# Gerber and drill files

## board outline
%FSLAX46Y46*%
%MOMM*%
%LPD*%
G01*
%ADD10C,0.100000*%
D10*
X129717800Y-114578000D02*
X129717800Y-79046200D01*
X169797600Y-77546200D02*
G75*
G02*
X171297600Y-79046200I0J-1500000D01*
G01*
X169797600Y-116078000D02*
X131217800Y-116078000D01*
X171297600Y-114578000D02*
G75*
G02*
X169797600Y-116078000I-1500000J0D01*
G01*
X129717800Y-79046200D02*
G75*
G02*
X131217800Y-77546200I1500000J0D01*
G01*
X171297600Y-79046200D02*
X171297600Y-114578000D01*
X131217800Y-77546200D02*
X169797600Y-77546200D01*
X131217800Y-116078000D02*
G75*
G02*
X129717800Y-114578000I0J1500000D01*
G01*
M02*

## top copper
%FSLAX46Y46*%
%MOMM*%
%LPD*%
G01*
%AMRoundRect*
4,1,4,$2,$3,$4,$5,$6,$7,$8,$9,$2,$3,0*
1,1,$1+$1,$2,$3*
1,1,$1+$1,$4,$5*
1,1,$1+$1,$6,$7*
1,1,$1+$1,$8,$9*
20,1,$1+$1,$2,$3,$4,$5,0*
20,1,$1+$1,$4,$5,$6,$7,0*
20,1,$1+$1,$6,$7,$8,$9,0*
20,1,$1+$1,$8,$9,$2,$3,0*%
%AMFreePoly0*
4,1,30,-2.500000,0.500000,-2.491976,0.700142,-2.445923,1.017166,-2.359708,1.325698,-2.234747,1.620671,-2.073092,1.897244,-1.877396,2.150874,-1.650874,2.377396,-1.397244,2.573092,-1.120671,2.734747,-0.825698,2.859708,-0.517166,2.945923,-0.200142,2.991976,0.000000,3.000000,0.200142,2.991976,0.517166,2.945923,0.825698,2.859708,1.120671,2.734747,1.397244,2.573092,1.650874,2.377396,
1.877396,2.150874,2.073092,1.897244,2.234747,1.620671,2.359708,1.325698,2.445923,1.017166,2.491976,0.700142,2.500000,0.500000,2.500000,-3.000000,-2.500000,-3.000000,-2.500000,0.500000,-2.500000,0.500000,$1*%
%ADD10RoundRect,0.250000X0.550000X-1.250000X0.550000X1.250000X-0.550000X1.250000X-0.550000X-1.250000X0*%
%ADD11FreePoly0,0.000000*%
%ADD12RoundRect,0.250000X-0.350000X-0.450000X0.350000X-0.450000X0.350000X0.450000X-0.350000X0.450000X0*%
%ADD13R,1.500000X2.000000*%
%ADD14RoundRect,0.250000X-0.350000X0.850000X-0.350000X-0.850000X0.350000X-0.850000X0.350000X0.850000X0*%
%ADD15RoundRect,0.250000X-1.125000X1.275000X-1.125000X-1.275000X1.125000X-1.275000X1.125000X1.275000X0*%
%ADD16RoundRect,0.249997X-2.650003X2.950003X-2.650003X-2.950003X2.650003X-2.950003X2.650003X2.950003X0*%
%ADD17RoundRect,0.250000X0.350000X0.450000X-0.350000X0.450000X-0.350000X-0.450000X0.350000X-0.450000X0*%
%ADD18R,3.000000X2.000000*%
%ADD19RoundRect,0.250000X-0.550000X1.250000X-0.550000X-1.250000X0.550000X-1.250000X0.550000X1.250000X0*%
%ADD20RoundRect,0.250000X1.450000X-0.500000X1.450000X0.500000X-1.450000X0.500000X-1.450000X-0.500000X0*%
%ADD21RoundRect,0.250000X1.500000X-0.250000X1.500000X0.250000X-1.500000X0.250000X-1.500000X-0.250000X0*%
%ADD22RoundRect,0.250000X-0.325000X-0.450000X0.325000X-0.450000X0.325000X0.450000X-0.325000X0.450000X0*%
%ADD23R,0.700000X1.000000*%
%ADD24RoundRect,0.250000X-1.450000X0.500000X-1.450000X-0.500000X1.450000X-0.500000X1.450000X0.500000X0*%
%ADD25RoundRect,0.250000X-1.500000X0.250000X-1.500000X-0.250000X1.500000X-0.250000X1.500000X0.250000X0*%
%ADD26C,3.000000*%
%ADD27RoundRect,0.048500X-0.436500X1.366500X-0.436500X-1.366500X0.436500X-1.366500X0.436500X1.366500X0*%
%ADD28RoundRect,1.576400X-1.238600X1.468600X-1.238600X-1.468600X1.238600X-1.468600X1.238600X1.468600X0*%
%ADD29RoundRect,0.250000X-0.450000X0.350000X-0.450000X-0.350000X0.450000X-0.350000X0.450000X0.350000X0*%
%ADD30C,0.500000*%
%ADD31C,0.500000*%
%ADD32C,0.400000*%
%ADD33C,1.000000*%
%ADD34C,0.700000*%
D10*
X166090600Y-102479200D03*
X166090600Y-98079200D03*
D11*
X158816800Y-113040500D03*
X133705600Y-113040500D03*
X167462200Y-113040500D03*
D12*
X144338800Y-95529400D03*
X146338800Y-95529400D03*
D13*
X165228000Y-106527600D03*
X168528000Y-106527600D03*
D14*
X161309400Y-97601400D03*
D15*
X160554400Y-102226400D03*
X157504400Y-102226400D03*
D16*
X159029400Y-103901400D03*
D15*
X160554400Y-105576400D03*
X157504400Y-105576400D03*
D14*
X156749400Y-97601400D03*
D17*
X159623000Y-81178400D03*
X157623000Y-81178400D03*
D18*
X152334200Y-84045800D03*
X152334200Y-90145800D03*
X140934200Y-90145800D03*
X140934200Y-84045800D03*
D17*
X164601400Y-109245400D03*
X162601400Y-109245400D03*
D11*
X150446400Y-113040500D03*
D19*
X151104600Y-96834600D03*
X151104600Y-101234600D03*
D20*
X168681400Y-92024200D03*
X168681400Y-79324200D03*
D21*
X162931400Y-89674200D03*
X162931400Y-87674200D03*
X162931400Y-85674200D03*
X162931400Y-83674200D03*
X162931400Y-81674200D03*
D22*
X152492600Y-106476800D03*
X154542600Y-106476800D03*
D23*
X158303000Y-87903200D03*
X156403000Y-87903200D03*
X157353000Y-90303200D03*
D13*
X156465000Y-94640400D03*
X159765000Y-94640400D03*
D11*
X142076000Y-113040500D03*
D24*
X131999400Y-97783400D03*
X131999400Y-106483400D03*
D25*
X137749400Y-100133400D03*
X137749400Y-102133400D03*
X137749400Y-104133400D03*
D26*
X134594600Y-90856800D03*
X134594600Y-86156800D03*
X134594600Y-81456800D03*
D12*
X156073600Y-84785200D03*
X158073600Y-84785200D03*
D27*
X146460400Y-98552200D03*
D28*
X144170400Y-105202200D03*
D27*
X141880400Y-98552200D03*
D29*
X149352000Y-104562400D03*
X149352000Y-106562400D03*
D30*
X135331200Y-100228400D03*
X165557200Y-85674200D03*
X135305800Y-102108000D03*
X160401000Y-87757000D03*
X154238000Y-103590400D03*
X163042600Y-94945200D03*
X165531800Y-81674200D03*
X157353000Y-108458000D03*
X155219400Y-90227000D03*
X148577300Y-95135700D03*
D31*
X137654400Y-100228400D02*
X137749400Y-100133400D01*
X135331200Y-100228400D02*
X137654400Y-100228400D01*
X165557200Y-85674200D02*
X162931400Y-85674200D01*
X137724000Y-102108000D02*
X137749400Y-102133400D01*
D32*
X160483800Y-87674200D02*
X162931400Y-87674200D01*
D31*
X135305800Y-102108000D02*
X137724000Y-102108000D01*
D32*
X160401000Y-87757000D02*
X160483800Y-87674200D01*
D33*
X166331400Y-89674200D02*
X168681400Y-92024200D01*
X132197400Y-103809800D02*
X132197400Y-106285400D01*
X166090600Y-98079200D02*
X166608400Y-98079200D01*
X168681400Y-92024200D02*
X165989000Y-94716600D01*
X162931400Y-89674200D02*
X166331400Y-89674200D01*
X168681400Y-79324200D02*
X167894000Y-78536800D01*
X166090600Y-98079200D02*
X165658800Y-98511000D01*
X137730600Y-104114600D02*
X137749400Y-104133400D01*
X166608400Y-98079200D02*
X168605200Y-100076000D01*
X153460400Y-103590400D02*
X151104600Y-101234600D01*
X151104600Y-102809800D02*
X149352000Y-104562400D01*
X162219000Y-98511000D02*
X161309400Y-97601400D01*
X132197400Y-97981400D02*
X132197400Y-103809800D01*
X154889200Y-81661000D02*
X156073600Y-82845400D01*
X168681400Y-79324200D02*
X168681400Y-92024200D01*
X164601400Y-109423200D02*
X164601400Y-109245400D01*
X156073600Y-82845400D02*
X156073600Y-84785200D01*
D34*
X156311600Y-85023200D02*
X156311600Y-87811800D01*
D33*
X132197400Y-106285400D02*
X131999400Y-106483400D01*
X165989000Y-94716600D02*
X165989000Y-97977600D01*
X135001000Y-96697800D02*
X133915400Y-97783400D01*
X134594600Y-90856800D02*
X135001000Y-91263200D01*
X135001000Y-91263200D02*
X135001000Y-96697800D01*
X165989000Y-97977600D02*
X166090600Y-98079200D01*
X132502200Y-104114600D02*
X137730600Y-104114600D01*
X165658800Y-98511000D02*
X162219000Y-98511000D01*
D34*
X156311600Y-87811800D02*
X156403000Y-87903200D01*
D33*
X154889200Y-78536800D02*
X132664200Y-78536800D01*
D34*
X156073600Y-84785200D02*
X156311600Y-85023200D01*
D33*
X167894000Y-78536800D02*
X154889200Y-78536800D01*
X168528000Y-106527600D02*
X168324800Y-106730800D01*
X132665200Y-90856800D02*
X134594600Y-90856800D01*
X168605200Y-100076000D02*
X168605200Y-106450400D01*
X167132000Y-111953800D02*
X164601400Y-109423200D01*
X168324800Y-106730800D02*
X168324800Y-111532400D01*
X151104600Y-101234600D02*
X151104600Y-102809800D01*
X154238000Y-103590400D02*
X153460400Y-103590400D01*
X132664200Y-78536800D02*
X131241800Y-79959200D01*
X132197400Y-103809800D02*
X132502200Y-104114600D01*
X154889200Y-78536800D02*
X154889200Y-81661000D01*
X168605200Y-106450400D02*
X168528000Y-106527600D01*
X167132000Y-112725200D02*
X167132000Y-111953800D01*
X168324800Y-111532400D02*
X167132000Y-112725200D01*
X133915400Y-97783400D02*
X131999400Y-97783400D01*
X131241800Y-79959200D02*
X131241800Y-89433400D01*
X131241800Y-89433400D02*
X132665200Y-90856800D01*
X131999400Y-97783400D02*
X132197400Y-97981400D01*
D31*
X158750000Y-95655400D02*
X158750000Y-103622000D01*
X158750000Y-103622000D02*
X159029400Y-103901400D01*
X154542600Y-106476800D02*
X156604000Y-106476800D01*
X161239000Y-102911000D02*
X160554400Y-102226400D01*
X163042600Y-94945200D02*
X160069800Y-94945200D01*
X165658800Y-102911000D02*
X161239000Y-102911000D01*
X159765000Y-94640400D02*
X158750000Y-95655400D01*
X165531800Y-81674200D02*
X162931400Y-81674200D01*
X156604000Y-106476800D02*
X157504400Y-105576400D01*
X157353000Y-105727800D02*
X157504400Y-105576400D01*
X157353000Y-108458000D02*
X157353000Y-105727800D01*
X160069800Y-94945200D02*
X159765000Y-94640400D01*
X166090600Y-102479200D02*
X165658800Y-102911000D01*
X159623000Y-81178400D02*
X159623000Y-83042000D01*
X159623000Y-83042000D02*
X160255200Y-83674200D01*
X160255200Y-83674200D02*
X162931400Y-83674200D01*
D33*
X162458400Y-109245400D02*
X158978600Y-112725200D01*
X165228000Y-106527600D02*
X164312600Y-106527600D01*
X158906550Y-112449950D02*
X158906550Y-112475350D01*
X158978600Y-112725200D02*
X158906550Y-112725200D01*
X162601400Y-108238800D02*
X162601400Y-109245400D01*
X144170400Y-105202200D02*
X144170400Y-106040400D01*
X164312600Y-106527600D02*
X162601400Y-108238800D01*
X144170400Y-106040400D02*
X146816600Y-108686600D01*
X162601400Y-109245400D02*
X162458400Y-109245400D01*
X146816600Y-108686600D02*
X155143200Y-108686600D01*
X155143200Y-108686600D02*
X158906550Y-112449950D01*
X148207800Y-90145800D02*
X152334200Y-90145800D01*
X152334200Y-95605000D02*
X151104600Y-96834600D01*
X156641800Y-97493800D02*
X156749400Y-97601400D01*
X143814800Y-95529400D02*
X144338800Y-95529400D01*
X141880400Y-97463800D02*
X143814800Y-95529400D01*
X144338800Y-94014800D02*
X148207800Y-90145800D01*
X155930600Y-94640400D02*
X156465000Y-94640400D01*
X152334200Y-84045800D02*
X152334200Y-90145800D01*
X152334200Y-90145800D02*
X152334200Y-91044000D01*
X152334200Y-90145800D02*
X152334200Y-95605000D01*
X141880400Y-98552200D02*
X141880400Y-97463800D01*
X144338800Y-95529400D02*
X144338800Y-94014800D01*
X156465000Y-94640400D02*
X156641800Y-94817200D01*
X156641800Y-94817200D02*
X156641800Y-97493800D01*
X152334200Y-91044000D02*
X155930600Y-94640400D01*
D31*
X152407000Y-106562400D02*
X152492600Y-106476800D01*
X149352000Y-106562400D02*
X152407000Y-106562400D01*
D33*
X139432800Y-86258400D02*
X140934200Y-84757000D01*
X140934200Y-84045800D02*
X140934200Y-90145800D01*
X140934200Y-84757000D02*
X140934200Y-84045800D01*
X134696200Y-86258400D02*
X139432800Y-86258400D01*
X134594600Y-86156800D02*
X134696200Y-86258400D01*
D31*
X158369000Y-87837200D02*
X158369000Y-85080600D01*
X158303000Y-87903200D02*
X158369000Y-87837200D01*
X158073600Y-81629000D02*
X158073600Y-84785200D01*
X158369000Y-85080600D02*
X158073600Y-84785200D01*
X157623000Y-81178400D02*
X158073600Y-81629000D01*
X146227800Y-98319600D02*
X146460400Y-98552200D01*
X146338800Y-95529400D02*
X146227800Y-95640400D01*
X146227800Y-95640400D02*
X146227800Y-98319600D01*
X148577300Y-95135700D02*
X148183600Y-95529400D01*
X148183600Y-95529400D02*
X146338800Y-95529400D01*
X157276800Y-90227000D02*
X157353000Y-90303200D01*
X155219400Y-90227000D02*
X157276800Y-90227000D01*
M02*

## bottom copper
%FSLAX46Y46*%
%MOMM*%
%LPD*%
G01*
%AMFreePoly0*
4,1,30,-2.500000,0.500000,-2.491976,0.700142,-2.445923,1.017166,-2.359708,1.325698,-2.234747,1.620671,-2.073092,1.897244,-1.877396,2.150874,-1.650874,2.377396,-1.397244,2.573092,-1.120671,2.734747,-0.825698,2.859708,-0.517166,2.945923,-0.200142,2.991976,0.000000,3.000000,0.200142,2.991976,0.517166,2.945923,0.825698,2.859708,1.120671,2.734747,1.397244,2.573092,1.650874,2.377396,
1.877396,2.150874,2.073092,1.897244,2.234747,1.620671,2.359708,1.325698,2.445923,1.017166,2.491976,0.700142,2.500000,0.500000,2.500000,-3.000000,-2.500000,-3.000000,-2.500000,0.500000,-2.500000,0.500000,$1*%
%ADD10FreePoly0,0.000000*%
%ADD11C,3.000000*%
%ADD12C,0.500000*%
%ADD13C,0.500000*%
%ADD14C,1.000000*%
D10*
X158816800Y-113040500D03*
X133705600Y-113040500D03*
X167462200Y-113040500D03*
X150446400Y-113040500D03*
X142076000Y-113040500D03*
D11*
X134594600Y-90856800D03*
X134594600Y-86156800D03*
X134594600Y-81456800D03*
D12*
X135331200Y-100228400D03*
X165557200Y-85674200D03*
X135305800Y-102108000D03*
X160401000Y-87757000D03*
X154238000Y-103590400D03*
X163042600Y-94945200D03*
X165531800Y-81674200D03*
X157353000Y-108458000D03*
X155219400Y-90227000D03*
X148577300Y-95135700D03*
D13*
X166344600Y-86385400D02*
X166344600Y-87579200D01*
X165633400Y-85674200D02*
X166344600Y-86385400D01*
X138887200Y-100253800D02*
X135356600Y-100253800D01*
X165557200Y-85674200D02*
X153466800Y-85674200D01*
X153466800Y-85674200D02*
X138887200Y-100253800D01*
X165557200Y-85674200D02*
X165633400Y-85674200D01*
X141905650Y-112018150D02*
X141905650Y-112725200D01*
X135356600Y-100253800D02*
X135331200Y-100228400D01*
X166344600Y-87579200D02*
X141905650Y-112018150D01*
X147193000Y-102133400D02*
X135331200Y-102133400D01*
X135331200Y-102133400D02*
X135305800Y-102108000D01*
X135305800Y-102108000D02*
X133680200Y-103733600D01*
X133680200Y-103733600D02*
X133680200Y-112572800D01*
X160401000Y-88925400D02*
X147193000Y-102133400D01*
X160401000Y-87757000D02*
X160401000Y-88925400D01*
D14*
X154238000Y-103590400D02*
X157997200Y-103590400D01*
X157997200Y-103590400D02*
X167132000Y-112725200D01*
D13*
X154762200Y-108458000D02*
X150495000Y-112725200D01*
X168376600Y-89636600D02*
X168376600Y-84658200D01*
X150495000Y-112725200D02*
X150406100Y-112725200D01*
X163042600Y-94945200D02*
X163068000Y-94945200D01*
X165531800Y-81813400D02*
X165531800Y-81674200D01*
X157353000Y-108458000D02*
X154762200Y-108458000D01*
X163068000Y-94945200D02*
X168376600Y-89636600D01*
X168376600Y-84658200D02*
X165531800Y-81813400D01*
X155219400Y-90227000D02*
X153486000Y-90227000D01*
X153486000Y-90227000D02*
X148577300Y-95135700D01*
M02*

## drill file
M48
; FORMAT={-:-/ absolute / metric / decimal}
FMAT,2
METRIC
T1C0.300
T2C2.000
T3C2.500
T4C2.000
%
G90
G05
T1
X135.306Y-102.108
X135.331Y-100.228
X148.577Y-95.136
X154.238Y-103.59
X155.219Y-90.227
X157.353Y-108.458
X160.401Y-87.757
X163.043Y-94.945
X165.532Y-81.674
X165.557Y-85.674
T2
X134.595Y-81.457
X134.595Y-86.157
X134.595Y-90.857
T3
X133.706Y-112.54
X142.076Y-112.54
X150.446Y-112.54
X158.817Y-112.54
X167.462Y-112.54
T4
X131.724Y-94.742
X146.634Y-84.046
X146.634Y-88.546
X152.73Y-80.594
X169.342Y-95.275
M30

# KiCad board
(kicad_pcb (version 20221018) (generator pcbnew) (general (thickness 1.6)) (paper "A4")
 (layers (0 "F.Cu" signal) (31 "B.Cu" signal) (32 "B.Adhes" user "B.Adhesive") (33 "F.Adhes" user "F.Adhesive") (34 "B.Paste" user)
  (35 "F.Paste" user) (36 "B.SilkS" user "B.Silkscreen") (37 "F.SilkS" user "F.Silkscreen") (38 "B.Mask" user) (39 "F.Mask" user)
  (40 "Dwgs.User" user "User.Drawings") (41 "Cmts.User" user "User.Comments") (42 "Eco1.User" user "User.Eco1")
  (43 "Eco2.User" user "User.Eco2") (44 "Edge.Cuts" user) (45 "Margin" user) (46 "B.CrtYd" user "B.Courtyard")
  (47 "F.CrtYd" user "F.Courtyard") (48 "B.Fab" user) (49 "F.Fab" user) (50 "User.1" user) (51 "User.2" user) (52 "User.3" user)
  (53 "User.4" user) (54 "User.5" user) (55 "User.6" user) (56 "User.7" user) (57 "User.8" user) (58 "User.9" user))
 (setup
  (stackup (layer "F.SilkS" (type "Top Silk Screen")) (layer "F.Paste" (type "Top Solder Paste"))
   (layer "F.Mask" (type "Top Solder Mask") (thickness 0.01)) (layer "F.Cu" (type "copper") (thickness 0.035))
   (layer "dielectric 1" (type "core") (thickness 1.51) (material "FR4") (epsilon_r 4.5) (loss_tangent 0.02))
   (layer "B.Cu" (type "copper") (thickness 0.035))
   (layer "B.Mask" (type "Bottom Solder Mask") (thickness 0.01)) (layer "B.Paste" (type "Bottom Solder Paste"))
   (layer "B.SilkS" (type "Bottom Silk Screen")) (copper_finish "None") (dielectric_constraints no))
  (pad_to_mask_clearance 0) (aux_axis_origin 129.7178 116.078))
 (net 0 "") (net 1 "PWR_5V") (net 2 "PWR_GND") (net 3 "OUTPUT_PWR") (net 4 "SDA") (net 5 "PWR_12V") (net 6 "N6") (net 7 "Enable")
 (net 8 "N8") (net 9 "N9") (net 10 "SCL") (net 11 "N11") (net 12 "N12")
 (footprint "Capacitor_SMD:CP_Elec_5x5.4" (layer "F.Cu") (at 166.0906 100.2792 90)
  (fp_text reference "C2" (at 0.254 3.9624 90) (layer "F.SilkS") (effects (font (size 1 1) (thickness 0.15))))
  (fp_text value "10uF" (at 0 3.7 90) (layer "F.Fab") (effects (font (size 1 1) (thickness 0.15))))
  (pad "1" smd roundrect (at -2.2 0 90) (size 3 1.6) (layers "F.Cu" "F.Paste" "F.Mask") (roundrect_rratio 0.15625) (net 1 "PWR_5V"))
  (pad "2" smd roundrect (at 2.2 0 90) (size 3 1.6) (layers "F.Cu" "F.Paste" "F.Mask") (roundrect_rratio 0.15625) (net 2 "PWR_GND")))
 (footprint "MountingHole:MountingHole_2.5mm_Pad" (layer "F.Cu") (at 158.8168 112.5405)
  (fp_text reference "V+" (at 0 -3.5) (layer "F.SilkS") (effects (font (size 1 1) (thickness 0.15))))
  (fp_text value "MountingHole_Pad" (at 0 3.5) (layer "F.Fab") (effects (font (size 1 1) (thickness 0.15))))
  (pad "1" thru_hole roundrect (at 0 0) (size 5 6) (drill 2.5 (offset 0 0.5)) (layers "*.Cu" "*.Mask") (roundrect_rratio 0.5)
   (chamfer_ratio 0) (chamfer bottom_left bottom_right) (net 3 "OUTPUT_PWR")))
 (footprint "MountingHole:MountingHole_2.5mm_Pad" (layer "F.Cu") (at 133.7056 112.5405)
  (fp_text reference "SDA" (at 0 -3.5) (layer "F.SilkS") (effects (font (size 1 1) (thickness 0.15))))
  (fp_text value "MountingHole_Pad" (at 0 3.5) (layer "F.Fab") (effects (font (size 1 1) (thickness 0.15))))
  (pad "1" thru_hole roundrect (at 0 0) (size 5 6) (drill 2.5 (offset 0 0.5)) (layers "*.Cu" "*.Mask") (roundrect_rratio 0.5)
   (chamfer_ratio 0) (chamfer bottom_left bottom_right) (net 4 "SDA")))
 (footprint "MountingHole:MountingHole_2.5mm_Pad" (layer "F.Cu") (at 167.4622 112.5405)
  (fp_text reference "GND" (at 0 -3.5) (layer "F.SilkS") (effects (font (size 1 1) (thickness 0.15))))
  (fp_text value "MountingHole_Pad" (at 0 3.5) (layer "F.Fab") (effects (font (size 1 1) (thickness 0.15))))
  (pad "1" thru_hole roundrect (at 0 0) (size 5 6) (drill 2.5 (offset 0 0.5)) (layers "*.Cu" "*.Mask") (roundrect_rratio 0.5)
   (chamfer_ratio 0) (chamfer bottom_left bottom_right) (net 2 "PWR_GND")))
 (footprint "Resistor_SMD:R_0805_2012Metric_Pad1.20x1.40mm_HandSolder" (layer "F.Cu") (at 145.3388 95.5294)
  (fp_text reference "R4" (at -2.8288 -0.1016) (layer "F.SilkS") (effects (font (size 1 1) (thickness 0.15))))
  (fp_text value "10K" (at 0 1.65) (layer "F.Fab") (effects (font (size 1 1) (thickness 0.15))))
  (pad "1" smd roundrect (at -1 0) (size 1.2 1.4) (layers "F.Cu" "F.Paste" "F.Mask") (roundrect_rratio 0.2083333333) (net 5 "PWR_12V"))
  (pad "2" smd roundrect (at 1 0) (size 1.2 1.4) (layers "F.Cu" "F.Paste" "F.Mask") (roundrect_rratio 0.2083333333) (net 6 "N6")))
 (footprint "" (layer "F.Cu") (at 131.7244 94.742)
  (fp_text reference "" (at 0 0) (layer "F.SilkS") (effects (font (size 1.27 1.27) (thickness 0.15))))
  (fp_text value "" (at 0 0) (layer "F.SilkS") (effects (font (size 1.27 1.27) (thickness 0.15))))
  (pad "" np_thru_hole circle (at 0 0) (size 2 2) (drill 2) (layers "F&B.Cu" "*.Mask")))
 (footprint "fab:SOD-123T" (layer "F.Cu") (at 166.878 106.5276)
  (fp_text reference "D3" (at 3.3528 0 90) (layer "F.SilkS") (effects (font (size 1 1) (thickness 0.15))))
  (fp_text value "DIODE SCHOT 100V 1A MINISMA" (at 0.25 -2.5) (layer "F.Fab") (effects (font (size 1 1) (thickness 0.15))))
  (pad "1" smd rect (at -1.65 0) (size 1.5 2) (layers "F.Cu" "F.Paste" "F.Mask") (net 3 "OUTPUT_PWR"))
  (pad "2" smd rect (at 1.65 0) (size 1.5 2) (layers "F.Cu" "F.Paste" "F.Mask") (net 2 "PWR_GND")))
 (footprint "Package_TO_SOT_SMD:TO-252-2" (layer "F.Cu") (at 159.0294 102.6414 -90)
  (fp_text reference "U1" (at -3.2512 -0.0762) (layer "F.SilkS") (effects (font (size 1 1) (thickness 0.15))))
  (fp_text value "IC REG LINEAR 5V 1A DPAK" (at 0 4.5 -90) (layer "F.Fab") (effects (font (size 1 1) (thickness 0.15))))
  (pad "1" smd roundrect (at -5.04 -2.28 270) (size 2.2 1.2) (layers "F.Cu" "F.Paste" "F.Mask") (roundrect_rratio 0.2083333333)
   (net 2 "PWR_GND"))
  (pad "2" smd roundrect (at -0.415 -1.525 270) (size 3.05 2.75) (layers "F.Cu" "F.Paste") (roundrect_rratio 0.09090909091) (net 1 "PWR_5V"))
  (pad "2" smd roundrect (at -0.415 1.525 270) (size 3.05 2.75) (layers "F.Cu" "F.Paste") (roundrect_rratio 0.09090909091) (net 1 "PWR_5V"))
  (pad "2" smd roundrect (at 1.26 0 270) (size 6.4 5.8) (layers "F.Cu" "F.Mask") (roundrect_rratio 0.04310293103) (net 1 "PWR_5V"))
  (pad "2" smd roundrect (at 2.935 -1.525 270) (size 3.05 2.75) (layers "F.Cu" "F.Paste") (roundrect_rratio 0.09090909091) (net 1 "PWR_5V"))
  (pad "2" smd roundrect (at 2.935 1.525 270) (size 3.05 2.75) (layers "F.Cu" "F.Paste") (roundrect_rratio 0.09090909091) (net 1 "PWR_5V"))
  (pad "3" smd roundrect (at -5.04 2.28 270) (size 2.2 1.2) (layers "F.Cu" "F.Paste" "F.Mask") (roundrect_rratio 0.2083333333)
   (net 5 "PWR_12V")))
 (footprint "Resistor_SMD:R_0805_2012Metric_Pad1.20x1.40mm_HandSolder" (layer "F.Cu") (at 158.623 81.1784 180)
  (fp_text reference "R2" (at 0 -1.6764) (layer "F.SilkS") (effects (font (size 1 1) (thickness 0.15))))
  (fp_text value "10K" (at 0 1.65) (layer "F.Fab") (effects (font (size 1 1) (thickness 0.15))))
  (pad "1" smd roundrect (at -1 0 180) (size 1.2 1.4) (layers "F.Cu" "F.Paste" "F.Mask") (roundrect_rratio 0.2083333333) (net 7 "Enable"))
  (pad "2" smd roundrect (at 1 0 180) (size 1.2 1.4) (layers "F.Cu" "F.Paste" "F.Mask") (roundrect_rratio 0.2083333333) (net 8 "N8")))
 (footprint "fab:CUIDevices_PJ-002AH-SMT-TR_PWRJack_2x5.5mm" (layer "F.Cu") (at 146.6342 87.0458 -90)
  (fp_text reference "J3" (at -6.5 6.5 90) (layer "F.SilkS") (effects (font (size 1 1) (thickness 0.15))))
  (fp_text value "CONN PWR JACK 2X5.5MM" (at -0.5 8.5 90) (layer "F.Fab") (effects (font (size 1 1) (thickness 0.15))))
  (pad "" np_thru_hole circle (at -3 0) (size 2 2) (drill 2) (layers "F&B.Cu" "*.Mask"))
  (pad "" np_thru_hole circle (at 1.5 0) (size 2 2) (drill 2) (layers "F&B.Cu" "*.Mask"))
  (pad "1" smd rect (at -3 -5.7) (size 3 2) (layers "F.Cu" "F.Paste" "F.Mask") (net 5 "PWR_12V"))
  (pad "1" smd rect (at 3.1 -5.7) (size 3 2) (layers "F.Cu" "F.Paste" "F.Mask") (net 5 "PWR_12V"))
  (pad "2" smd rect (at 3.1 5.7) (size 3 2) (layers "F.Cu" "F.Paste" "F.Mask") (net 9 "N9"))
  (pad "3" smd rect (at -3 5.7) (size 3 2) (layers "F.Cu" "F.Paste" "F.Mask") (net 9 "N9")))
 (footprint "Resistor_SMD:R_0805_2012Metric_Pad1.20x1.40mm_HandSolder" (layer "F.Cu") (at 163.6014 109.2454 180)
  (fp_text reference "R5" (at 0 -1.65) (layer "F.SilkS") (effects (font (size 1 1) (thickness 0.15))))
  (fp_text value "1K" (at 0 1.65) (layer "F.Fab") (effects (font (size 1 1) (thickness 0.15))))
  (pad "1" smd roundrect (at -1 0 180) (size 1.2 1.4) (layers "F.Cu" "F.Paste" "F.Mask") (roundrect_rratio 0.2083333333) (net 2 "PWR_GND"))
  (pad "2" smd roundrect (at 1 0 180) (size 1.2 1.4) (layers "F.Cu" "F.Paste" "F.Mask") (roundrect_rratio 0.2083333333) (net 3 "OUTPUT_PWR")))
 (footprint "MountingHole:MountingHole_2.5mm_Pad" (layer "F.Cu") (at 150.4464 112.5405)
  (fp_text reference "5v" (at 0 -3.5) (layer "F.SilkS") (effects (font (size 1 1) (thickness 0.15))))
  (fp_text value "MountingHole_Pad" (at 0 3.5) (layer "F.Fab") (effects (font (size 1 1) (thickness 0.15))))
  (pad "1" thru_hole roundrect (at 0 0) (size 5 6) (drill 2.5 (offset 0 0.5)) (layers "*.Cu" "*.Mask") (roundrect_rratio 0.5)
   (chamfer_ratio 0) (chamfer bottom_left bottom_right) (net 1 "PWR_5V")))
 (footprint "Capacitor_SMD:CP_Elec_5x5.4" (layer "F.Cu") (at 151.1046 99.0346 -90)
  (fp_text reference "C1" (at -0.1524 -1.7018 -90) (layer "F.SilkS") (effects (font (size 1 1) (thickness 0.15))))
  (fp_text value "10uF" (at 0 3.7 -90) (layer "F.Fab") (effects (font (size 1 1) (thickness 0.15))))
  (pad "1" smd roundrect (at -2.2 0 270) (size 3 1.6) (layers "F.Cu" "F.Paste" "F.Mask") (roundrect_rratio 0.15625) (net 5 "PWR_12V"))
  (pad "2" smd roundrect (at 2.2 0 270) (size 3 1.6) (layers "F.Cu" "F.Paste" "F.Mask") (roundrect_rratio 0.15625) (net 2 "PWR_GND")))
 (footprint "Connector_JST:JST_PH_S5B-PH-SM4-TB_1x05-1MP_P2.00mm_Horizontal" (layer "F.Cu") (at 165.7814 85.6742 90)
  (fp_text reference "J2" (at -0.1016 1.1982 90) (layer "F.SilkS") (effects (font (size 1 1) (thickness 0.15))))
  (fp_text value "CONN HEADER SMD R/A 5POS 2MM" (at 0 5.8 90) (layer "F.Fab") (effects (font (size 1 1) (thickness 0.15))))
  (pad "" smd roundrect (at -6.35 2.9 90) (size 1.5 3.4) (layers "F.Cu" "F.Paste" "F.Mask") (roundrect_rratio 0.1666666667)
   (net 2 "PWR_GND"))
  (pad "" smd roundrect (at 6.35 2.9 90) (size 1.5 3.4) (layers "F.Cu" "F.Paste" "F.Mask") (roundrect_rratio 0.1666666667) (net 2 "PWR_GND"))
  (pad "1" smd roundrect (at -4 -2.85 90) (size 1 3.5) (layers "F.Cu" "F.Paste" "F.Mask") (roundrect_rratio 0.25) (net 2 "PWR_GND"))
  (pad "2" smd roundrect (at -2 -2.85 90) (size 1 3.5) (layers "F.Cu" "F.Paste" "F.Mask") (roundrect_rratio 0.25) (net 4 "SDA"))
  (pad "3" smd roundrect (at 0 -2.85 90) (size 1 3.5) (layers "F.Cu" "F.Paste" "F.Mask") (roundrect_rratio 0.25) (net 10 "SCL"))
  (pad "4" smd roundrect (at 2 -2.85 90) (size 1 3.5) (layers "F.Cu" "F.Paste" "F.Mask") (roundrect_rratio 0.25) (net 7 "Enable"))
  (pad "5" smd roundrect (at 4 -2.85 90) (size 1 3.5) (layers "F.Cu" "F.Paste" "F.Mask") (roundrect_rratio 0.25) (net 1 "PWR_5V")))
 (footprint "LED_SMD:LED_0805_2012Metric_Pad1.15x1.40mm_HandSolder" (layer "F.Cu") (at 153.5176 106.4768)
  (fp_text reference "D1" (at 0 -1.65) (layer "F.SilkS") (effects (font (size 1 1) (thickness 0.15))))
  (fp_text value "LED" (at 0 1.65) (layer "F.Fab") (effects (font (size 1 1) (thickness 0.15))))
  (pad "1" smd roundrect (at -1.025 0) (size 1.15 1.4) (layers "F.Cu" "F.Paste" "F.Mask") (roundrect_rratio 0.2173913043) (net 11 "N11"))
  (pad "2" smd roundrect (at 1.025 0) (size 1.15 1.4) (layers "F.Cu" "F.Paste" "F.Mask") (roundrect_rratio 0.2173913043) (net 1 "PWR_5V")))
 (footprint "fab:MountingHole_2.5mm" (layer "F.Cu") (at 152.7302 80.5942)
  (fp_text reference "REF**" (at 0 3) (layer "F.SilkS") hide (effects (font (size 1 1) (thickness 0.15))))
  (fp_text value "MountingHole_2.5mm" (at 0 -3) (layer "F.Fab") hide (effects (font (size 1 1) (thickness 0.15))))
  (pad "" np_thru_hole circle (at 0 0) (size 2 2) (drill 2) (layers "*.Cu" "*.Mask")))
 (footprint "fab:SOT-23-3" (layer "F.Cu") (at 157.353 89.1032 -90)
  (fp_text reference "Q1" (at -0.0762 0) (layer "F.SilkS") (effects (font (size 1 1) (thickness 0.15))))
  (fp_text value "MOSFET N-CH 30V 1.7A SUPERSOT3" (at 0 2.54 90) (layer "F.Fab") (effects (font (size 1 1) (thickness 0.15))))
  (pad "1" smd rect (at -1.2 -0.95 270) (size 1 0.7) (layers "F.Cu" "F.Paste" "F.Mask") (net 8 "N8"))
  (pad "2" smd rect (at -1.2 0.95 270) (size 1 0.7) (layers "F.Cu" "F.Paste" "F.Mask") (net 2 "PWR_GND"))
  (pad "3" smd rect (at 1.2 0 270) (size 1 0.7) (layers "F.Cu" "F.Paste" "F.Mask") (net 6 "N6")))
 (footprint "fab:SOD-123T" (layer "F.Cu") (at 158.115 94.6404)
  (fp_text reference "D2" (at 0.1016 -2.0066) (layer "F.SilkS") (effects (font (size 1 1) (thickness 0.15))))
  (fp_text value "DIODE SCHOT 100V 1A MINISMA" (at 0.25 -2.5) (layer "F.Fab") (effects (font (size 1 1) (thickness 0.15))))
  (pad "1" smd rect (at -1.65 0) (size 1.5 2) (layers "F.Cu" "F.Paste" "F.Mask") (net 5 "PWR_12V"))
  (pad "2" smd rect (at 1.65 0) (size 1.5 2) (layers "F.Cu" "F.Paste" "F.Mask") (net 1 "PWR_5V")))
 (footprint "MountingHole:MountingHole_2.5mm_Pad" (layer "F.Cu") (at 142.076 112.5405)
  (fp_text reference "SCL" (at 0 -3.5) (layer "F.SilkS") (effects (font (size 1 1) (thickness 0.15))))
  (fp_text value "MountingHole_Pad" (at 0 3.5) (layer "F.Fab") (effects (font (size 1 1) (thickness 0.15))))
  (pad "1" thru_hole roundrect (at 0 0) (size 5 6) (drill 2.5 (offset 0 0.5)) (layers "*.Cu" "*.Mask") (roundrect_rratio 0.5)
   (chamfer_ratio 0) (chamfer bottom_left bottom_right) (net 10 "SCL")))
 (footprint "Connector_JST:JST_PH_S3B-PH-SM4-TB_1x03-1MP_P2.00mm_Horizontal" (layer "F.Cu") (at 134.8994 102.1334 -90)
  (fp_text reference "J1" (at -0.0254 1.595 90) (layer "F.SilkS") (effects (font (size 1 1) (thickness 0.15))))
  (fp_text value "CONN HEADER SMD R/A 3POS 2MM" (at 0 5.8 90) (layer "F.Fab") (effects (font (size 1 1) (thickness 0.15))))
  (pad "" smd roundrect (at -4.35 2.9 270) (size 1.5 3.4) (layers "F.Cu" "F.Paste" "F.Mask") (roundrect_rratio 0.1666666667)
   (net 2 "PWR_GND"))
  (pad "" smd roundrect (at 4.35 2.9 270) (size 1.5 3.4) (layers "F.Cu" "F.Paste" "F.Mask") (roundrect_rratio 0.1666666667)
   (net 2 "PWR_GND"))
  (pad "1" smd roundrect (at -2 -2.85 270) (size 1 3.5) (layers "F.Cu" "F.Paste" "F.Mask") (roundrect_rratio 0.25) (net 10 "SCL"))
  (pad "2" smd roundrect (at 0 -2.85 270) (size 1 3.5) (layers "F.Cu" "F.Paste" "F.Mask") (roundrect_rratio 0.25) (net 4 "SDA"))
  (pad "3" smd roundrect (at 2 -2.85 270) (size 1 3.5) (layers "F.Cu" "F.Paste" "F.Mask") (roundrect_rratio 0.25) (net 2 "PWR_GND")))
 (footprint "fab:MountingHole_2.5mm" (layer "F.Cu") (at 169.3418 95.2754)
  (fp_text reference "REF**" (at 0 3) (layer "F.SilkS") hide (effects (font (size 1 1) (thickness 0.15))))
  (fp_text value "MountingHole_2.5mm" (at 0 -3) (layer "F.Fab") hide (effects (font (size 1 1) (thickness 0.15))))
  (pad "" np_thru_hole circle (at 0 0) (size 2 2) (drill 2) (layers "F&B.Cu" "*.Mask")))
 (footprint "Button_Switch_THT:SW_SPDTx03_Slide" (layer "F.Cu") (at 134.5946 86.1568 90)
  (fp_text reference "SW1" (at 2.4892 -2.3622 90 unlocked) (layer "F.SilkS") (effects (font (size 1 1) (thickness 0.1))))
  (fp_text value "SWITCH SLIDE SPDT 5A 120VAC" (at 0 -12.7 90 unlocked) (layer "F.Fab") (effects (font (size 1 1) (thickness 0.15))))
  (pad "1" thru_hole circle (at -4.7 0 90) (size 3 3) (drill 2) (layers "*.Cu" "*.Mask") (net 2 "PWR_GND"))
  (pad "2" thru_hole circle (at 0 0 90) (size 3 3) (drill 2) (layers "*.Cu" "*.Mask") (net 9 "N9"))
  (pad "3" thru_hole circle (at 4.7 0 90) (size 3 3) (drill 2) (layers "*.Cu" "*.Mask") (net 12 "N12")))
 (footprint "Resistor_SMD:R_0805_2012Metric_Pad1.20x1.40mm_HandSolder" (layer "F.Cu") (at 157.0736 84.7852)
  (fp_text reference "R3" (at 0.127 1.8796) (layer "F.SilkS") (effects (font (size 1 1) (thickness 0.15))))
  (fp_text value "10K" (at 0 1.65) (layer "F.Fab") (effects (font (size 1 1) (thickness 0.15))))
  (pad "1" smd roundrect (at -1 0) (size 1.2 1.4) (layers "F.Cu" "F.Paste" "F.Mask") (roundrect_rratio 0.2083333333) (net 2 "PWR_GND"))
  (pad "2" smd roundrect (at 1 0) (size 1.2 1.4) (layers "F.Cu" "F.Paste" "F.Mask") (roundrect_rratio 0.2083333333) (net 8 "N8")))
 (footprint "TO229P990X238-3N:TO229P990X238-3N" (layer "F.Cu") (at 144.1704 102.6922 -90)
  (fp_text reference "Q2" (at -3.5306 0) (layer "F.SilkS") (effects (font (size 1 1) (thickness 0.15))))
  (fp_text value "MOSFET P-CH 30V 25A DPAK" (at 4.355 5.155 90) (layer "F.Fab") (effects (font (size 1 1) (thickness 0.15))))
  (pad "1" smd roundrect (at -4.14 -2.29 270) (size 2.83 0.97) (layers "F.Cu" "F.Paste" "F.Mask") (roundrect_rratio 0.05) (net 6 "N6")
   (solder_mask_margin 0.102))
  (pad "2" smd roundrect (at 2.51 0 270) (size 6.09 5.63) (layers "F.Cu" "F.Mask") (roundrect_rratio 0.28) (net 3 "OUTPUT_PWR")
   (solder_mask_margin 0.102))
  (pad "3" smd roundrect (at -4.14 2.29 270) (size 2.83 0.97) (layers "F.Cu" "F.Paste" "F.Mask") (roundrect_rratio 0.05) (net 5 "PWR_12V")
   (solder_mask_margin 0.102)))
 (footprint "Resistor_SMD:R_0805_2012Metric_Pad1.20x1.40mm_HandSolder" (layer "F.Cu") (at 149.352 105.5624 -90)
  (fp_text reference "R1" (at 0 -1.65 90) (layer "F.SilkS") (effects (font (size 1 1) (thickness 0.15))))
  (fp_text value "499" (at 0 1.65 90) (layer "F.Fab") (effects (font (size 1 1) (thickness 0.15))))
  (pad "1" smd roundrect (at -1 0 270) (size 1.2 1.4) (layers "F.Cu" "F.Paste" "F.Mask") (roundrect_rratio 0.2083333333) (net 2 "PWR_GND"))
  (pad "2" smd roundrect (at 1 0 270) (size 1.2 1.4) (layers "F.Cu" "F.Paste" "F.Mask") (roundrect_rratio 0.2083333333) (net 11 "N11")))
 (gr_line (start 129.7178 114.578) (end 129.7178 79.0462) (stroke (width 0.1) (type default)) (layer "Edge.Cuts"))
 (gr_arc (start 169.7976 77.5462) (mid 170.85826 77.98554) (end 171.2976 79.0462) (stroke (width 0.1) (type default)) (layer "Edge.Cuts"))
 (gr_line (start 169.7976 116.078) (end 131.2178 116.078) (stroke (width 0.1) (type default)) (layer "Edge.Cuts"))
 (gr_arc (start 171.2976 114.578) (mid 170.85826 115.63866) (end 169.7976 116.078) (stroke (width 0.1) (type default)) (layer "Edge.Cuts"))
 (gr_arc (start 129.7178 79.0462) (mid 130.15714 77.98554) (end 131.2178 77.5462) (stroke (width 0.1) (type default)) (layer "Edge.Cuts"))
 (gr_line (start 171.2976 79.0462) (end 171.2976 114.578) (stroke (width 0.1) (type default)) (layer "Edge.Cuts"))
 (gr_line (start 131.2178 77.5462) (end 169.7976 77.5462) (stroke (width 0.1) (type default)) (layer "Edge.Cuts"))
 (gr_arc (start 131.2178 116.078) (mid 130.15714 115.63866) (end 129.7178 114.578) (stroke (width 0.1) (type default)) (layer "Edge.Cuts"))
 (segment (start 137.6544 100.2284) (end 137.7494 100.1334) (width 0.5) (layer "F.Cu") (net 10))
 (segment (start 135.3312 100.2284) (end 137.6544 100.2284) (width 0.5) (layer "F.Cu") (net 10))
 (segment (start 165.5572 85.6742) (end 162.9314 85.6742) (width 0.5) (layer "F.Cu") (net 10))
 (via (at 135.3312 100.2284) (size 0.5) (drill 0.3) (layers "F.Cu" "B.Cu") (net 10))
 (via (at 165.5572 85.6742) (size 0.5) (drill 0.3) (layers "F.Cu" "B.Cu") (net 10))
 (segment (start 166.3446 86.3854) (end 166.3446 87.5792) (width 0.5) (layer "B.Cu") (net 10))
 (segment (start 165.6334 85.6742) (end 166.3446 86.3854) (width 0.5) (layer "B.Cu") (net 10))
 (segment (start 138.8872 100.2538) (end 135.3566 100.2538) (width 0.5) (layer "B.Cu") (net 10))
 (segment (start 165.5572 85.6742) (end 153.4668 85.6742) (width 0.5) (layer "B.Cu") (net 10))
 (segment (start 153.4668 85.6742) (end 138.8872 100.2538) (width 0.5) (layer "B.Cu") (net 10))
 (segment (start 165.5572 85.6742) (end 165.6334 85.6742) (width 0.5) (layer "B.Cu") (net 10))
 (segment (start 141.90565 112.01815) (end 141.90565 112.7252) (width 0.5) (layer "B.Cu") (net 10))
 (segment (start 135.3566 100.2538) (end 135.3312 100.2284) (width 0.5) (layer "B.Cu") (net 10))
 (segment (start 166.3446 87.5792) (end 141.90565 112.01815) (width 0.5) (layer "B.Cu") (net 10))
 (segment (start 137.724 102.108) (end 137.7494 102.1334) (width 0.5) (layer "F.Cu") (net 4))
 (segment (start 160.4838 87.6742) (end 162.9314 87.6742) (width 0.4) (layer "F.Cu") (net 4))
 (segment (start 135.3058 102.108) (end 137.724 102.108) (width 0.5) (layer "F.Cu") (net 4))
 (segment (start 160.401 87.757) (end 160.4838 87.6742) (width 0.4) (layer "F.Cu") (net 4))
 (via (at 135.3058 102.108) (size 0.5) (drill 0.3) (layers "F.Cu" "B.Cu") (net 4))
 (via (at 160.401 87.757) (size 0.5) (drill 0.3) (layers "F.Cu" "B.Cu") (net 4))
 (segment (start 147.193 102.1334) (end 135.3312 102.1334) (width 0.5) (layer "B.Cu") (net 4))
 (segment (start 135.3312 102.1334) (end 135.3058 102.108) (width 0.5) (layer "B.Cu") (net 4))
 (segment (start 135.3058 102.108) (end 133.6802 103.7336) (width 0.5) (layer "B.Cu") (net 4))
 (segment (start 133.6802 103.7336) (end 133.6802 112.5728) (width 0.5) (layer "B.Cu") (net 4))
 (segment (start 160.401 88.9254) (end 147.193 102.1334) (width 0.5) (layer "B.Cu") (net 4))
 (segment (start 160.401 87.757) (end 160.401 88.9254) (width 0.5) (layer "B.Cu") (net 4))
 (segment (start 166.3314 89.6742) (end 168.6814 92.0242) (width 1) (layer "F.Cu") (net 2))
 (segment (start 132.1974 103.8098) (end 132.1974 106.2854) (width 1) (layer "F.Cu") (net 2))
 (segment (start 166.0906 98.0792) (end 166.6084 98.0792) (width 1) (layer "F.Cu") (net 2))
 (segment (start 168.6814 92.0242) (end 165.989 94.7166) (width 1) (layer "F.Cu") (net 2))
 (segment (start 162.9314 89.6742) (end 166.3314 89.6742) (width 1) (layer "F.Cu") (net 2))
 (segment (start 168.6814 79.3242) (end 167.894 78.5368) (width 1) (layer "F.Cu") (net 2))
 (segment (start 166.0906 98.0792) (end 165.6588 98.511) (width 1) (layer "F.Cu") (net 2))
 (segment (start 137.7306 104.1146) (end 137.7494 104.1334) (width 1) (layer "F.Cu") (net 2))
 (segment (start 166.6084 98.0792) (end 168.6052 100.076) (width 1) (layer "F.Cu") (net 2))
 (segment (start 153.4604 103.5904) (end 151.1046 101.2346) (width 1) (layer "F.Cu") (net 2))
 (segment (start 151.1046 102.8098) (end 149.352 104.5624) (width 1) (layer "F.Cu") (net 2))
 (segment (start 162.219 98.511) (end 161.3094 97.6014) (width 1) (layer "F.Cu") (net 2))
 (segment (start 132.1974 97.9814) (end 132.1974 103.8098) (width 1) (layer "F.Cu") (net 2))
 (segment (start 154.8892 81.661) (end 156.0736 82.8454) (width 1) (layer "F.Cu") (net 2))
 (segment (start 168.6814 79.3242) (end 168.6814 92.0242) (width 1) (layer "F.Cu") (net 2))
 (segment (start 164.6014 109.4232) (end 164.6014 109.2454) (width 1) (layer "F.Cu") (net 2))
 (segment (start 156.0736 82.8454) (end 156.0736 84.7852) (width 1) (layer "F.Cu") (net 2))
 (segment (start 156.3116 85.0232) (end 156.3116 87.8118) (width 0.7) (layer "F.Cu") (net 2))
 (segment (start 132.1974 106.2854) (end 131.9994 106.4834) (width 1) (layer "F.Cu") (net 2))
 (segment (start 165.989 94.7166) (end 165.989 97.9776) (width 1) (layer "F.Cu") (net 2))
 (segment (start 135.001 96.6978) (end 133.9154 97.7834) (width 1) (layer "F.Cu") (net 2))
 (segment (start 134.5946 90.8568) (end 135.001 91.2632) (width 1) (layer "F.Cu") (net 2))
 (segment (start 135.001 91.2632) (end 135.001 96.6978) (width 1) (layer "F.Cu") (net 2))
 (segment (start 165.989 97.9776) (end 166.0906 98.0792) (width 1) (layer "F.Cu") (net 2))
 (segment (start 132.5022 104.1146) (end 137.7306 104.1146) (width 1) (layer "F.Cu") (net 2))
 (segment (start 165.6588 98.511) (end 162.219 98.511) (width 1) (layer "F.Cu") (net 2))
 (segment (start 156.3116 87.8118) (end 156.403 87.9032) (width 0.7) (layer "F.Cu") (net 2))
 (segment (start 154.8892 78.5368) (end 132.6642 78.5368) (width 1) (layer "F.Cu") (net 2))
 (segment (start 156.0736 84.7852) (end 156.3116 85.0232) (width 0.7) (layer "F.Cu") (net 2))
 (segment (start 167.894 78.5368) (end 154.8892 78.5368) (width 1) (layer "F.Cu") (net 2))
 (segment (start 168.528 106.5276) (end 168.3248 106.7308) (width 1) (layer "F.Cu") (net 2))
 (segment (start 132.6652 90.8568) (end 134.5946 90.8568) (width 1) (layer "F.Cu") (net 2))
 (segment (start 168.6052 100.076) (end 168.6052 106.4504) (width 1) (layer "F.Cu") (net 2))
 (segment (start 167.132 111.9538) (end 164.6014 109.4232) (width 1) (layer "F.Cu") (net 2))
 (segment (start 168.3248 106.7308) (end 168.3248 111.5324) (width 1) (layer "F.Cu") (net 2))
 (segment (start 151.1046 101.2346) (end 151.1046 102.8098) (width 1) (layer "F.Cu") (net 2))
 (segment (start 154.238 103.5904) (end 153.4604 103.5904) (width 1) (layer "F.Cu") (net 2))
 (segment (start 132.6642 78.5368) (end 131.2418 79.9592) (width 1) (layer "F.Cu") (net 2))
 (segment (start 132.1974 103.8098) (end 132.5022 104.1146) (width 1) (layer "F.Cu") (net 2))
 (segment (start 154.8892 78.5368) (end 154.8892 81.661) (width 1) (layer "F.Cu") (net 2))
 (segment (start 168.6052 106.4504) (end 168.528 106.5276) (width 1) (layer "F.Cu") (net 2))
 (segment (start 167.132 112.7252) (end 167.132 111.9538) (width 1) (layer "F.Cu") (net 2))
 (segment (start 168.3248 111.5324) (end 167.132 112.7252) (width 1) (layer "F.Cu") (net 2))
 (segment (start 133.9154 97.7834) (end 131.9994 97.7834) (width 1) (layer "F.Cu") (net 2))
 (segment (start 131.2418 79.9592) (end 131.2418 89.4334) (width 1) (layer "F.Cu") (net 2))
 (segment (start 131.2418 89.4334) (end 132.6652 90.8568) (width 1) (layer "F.Cu") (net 2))
 (segment (start 131.9994 97.7834) (end 132.1974 97.9814) (width 1) (layer "F.Cu") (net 2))
 (via (at 154.238 103.5904) (size 0.5) (drill 0.3) (layers "F.Cu" "B.Cu") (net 2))
 (segment (start 154.238 103.5904) (end 157.9972 103.5904) (width 1) (layer "B.Cu") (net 2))
 (segment (start 157.9972 103.5904) (end 167.132 112.7252) (width 1) (layer "B.Cu") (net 2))
 (segment (start 158.75 95.6554) (end 158.75 103.622) (width 0.5) (layer "F.Cu") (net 1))
 (segment (start 158.75 103.622) (end 159.0294 103.9014) (width 0.5) (layer "F.Cu") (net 1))
 (segment (start 154.5426 106.4768) (end 156.604 106.4768) (width 0.5) (layer "F.Cu") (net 1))
 (segment (start 161.239 102.911) (end 160.5544 102.2264) (width 0.5) (layer "F.Cu") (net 1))
 (segment (start 163.0426 94.9452) (end 160.0698 94.9452) (width 0.5) (layer "F.Cu") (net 1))
 (segment (start 165.6588 102.911) (end 161.239 102.911) (width 0.5) (layer "F.Cu") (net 1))
 (segment (start 159.765 94.6404) (end 158.75 95.6554) (width 0.5) (layer "F.Cu") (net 1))
 (segment (start 165.5318 81.6742) (end 162.9314 81.6742) (width 0.5) (layer "F.Cu") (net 1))
 (segment (start 156.604 106.4768) (end 157.5044 105.5764) (width 0.5) (layer "F.Cu") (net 1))
 (segment (start 157.353 105.7278) (end 157.5044 105.5764) (width 0.5) (layer "F.Cu") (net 1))
 (segment (start 157.353 108.458) (end 157.353 105.7278) (width 0.5) (layer "F.Cu") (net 1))
 (segment (start 160.0698 94.9452) (end 159.765 94.6404) (width 0.5) (layer "F.Cu") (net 1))
 (segment (start 166.0906 102.4792) (end 165.6588 102.911) (width 0.5) (layer "F.Cu") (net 1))
 (via (at 163.0426 94.9452) (size 0.5) (drill 0.3) (layers "F.Cu" "B.Cu") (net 1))
 (via (at 165.5318 81.6742) (size 0.5) (drill 0.3) (layers "F.Cu" "B.Cu") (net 1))
 (via (at 157.353 108.458) (size 0.5) (drill 0.3) (layers "F.Cu" "B.Cu") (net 1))
 (segment (start 154.7622 108.458) (end 150.495 112.7252) (width 0.5) (layer "B.Cu") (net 1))
 (segment (start 168.3766 89.6366) (end 168.3766 84.6582) (width 0.5) (layer "B.Cu") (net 1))
 (segment (start 150.495 112.7252) (end 150.4061 112.7252) (width 0.5) (layer "B.Cu") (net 1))
 (segment (start 163.0426 94.9452) (end 163.068 94.9452) (width 0.5) (layer "B.Cu") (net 1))
 (segment (start 165.5318 81.8134) (end 165.5318 81.6742) (width 0.5) (layer "B.Cu") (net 1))
 (segment (start 157.353 108.458) (end 154.7622 108.458) (width 0.5) (layer "B.Cu") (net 1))
 (segment (start 163.068 94.9452) (end 168.3766 89.6366) (width 0.5) (layer "B.Cu") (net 1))
 (segment (start 168.3766 84.6582) (end 165.5318 81.8134) (width 0.5) (layer "B.Cu") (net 1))
 (segment (start 159.623 81.1784) (end 159.623 83.042) (width 0.5) (layer "F.Cu") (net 7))
 (segment (start 159.623 83.042) (end 160.2552 83.6742) (width 0.5) (layer "F.Cu") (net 7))
 (segment (start 160.2552 83.6742) (end 162.9314 83.6742) (width 0.5) (layer "F.Cu") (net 7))
 (segment (start 162.4584 109.2454) (end 158.9786 112.7252) (width 1) (layer "F.Cu") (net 3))
 (segment (start 165.228 106.5276) (end 164.3126 106.5276) (width 1) (layer "F.Cu") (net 3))
 (segment (start 158.90655 112.44995) (end 158.90655 112.47535) (width 1) (layer "F.Cu") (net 3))
 (segment (start 158.9786 112.7252) (end 158.90655 112.7252) (width 1) (layer "F.Cu") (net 3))
 (segment (start 162.6014 108.2388) (end 162.6014 109.2454) (width 1) (layer "F.Cu") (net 3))
 (segment (start 144.1704 105.2022) (end 144.1704 106.0404) (width 1) (layer "F.Cu") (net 3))
 (segment (start 164.3126 106.5276) (end 162.6014 108.2388) (width 1) (layer "F.Cu") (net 3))
 (segment (start 144.1704 106.0404) (end 146.8166 108.6866) (width 1) (layer "F.Cu") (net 3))
 (segment (start 162.6014 109.2454) (end 162.4584 109.2454) (width 1) (layer "F.Cu") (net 3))
 (segment (start 146.8166 108.6866) (end 155.1432 108.6866) (width 1) (layer "F.Cu") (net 3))
 (segment (start 155.1432 108.6866) (end 158.90655 112.44995) (width 1) (layer "F.Cu") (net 3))
 (segment (start 148.2078 90.1458) (end 152.3342 90.1458) (width 1) (layer "F.Cu") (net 5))
 (segment (start 152.3342 95.605) (end 151.1046 96.8346) (width 1) (layer "F.Cu") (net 5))
 (segment (start 156.6418 97.4938) (end 156.7494 97.6014) (width 1) (layer "F.Cu") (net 5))
 (segment (start 143.8148 95.5294) (end 144.3388 95.5294) (width 1) (layer "F.Cu") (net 5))
 (segment (start 141.8804 97.4638) (end 143.8148 95.5294) (width 1) (layer "F.Cu") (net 5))
 (segment (start 144.3388 94.0148) (end 148.2078 90.1458) (width 1) (layer "F.Cu") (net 5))
 (segment (start 155.9306 94.6404) (end 156.465 94.6404) (width 1) (layer "F.Cu") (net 5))
 (segment (start 152.3342 84.0458) (end 152.3342 90.1458) (width 1) (layer "F.Cu") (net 5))
 (segment (start 152.3342 90.1458) (end 152.3342 91.044) (width 1) (layer "F.Cu") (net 5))
 (segment (start 152.3342 90.1458) (end 152.3342 95.605) (width 1) (layer "F.Cu") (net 5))
 (segment (start 141.8804 98.5522) (end 141.8804 97.4638) (width 1) (layer "F.Cu") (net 5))
 (segment (start 144.3388 95.5294) (end 144.3388 94.0148) (width 1) (layer "F.Cu") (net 5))
 (segment (start 156.465 94.6404) (end 156.6418 94.8172) (width 1) (layer "F.Cu") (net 5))
 (segment (start 156.6418 94.8172) (end 156.6418 97.4938) (width 1) (layer "F.Cu") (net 5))
 (segment (start 152.3342 91.044) (end 155.9306 94.6404) (width 1) (layer "F.Cu") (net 5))
 (segment (start 152.407 106.5624) (end 152.4926 106.4768) (width 0.5) (layer "F.Cu") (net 11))
 (segment (start 149.352 106.5624) (end 152.407 106.5624) (width 0.5) (layer "F.Cu") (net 11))
 (segment (start 139.4328 86.2584) (end 140.9342 84.757) (width 1) (layer "F.Cu") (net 9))
 (segment (start 140.9342 84.0458) (end 140.9342 90.1458) (width 1) (layer "F.Cu") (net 9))
 (segment (start 140.9342 84.757) (end 140.9342 84.0458) (width 1) (layer "F.Cu") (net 9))
 (segment (start 134.6962 86.2584) (end 139.4328 86.2584) (width 1) (layer "F.Cu") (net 9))
 (segment (start 134.5946 86.1568) (end 134.6962 86.2584) (width 1) (layer "F.Cu") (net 9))
 (segment (start 158.369 87.8372) (end 158.369 85.0806) (width 0.5) (layer "F.Cu") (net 8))
 (segment (start 158.303 87.9032) (end 158.369 87.8372) (width 0.5) (layer "F.Cu") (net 8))
 (segment (start 158.0736 81.629) (end 158.0736 84.7852) (width 0.5) (layer "F.Cu") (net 8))
 (segment (start 158.369 85.0806) (end 158.0736 84.7852) (width 0.5) (layer "F.Cu") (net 8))
 (segment (start 157.623 81.1784) (end 158.0736 81.629) (width 0.5) (layer "F.Cu") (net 8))
 (segment (start 146.2278 98.3196) (end 146.4604 98.5522) (width 0.5) (layer "F.Cu") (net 6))
 (segment (start 146.3388 95.5294) (end 146.2278 95.6404) (width 0.5) (layer "F.Cu") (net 6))
 (segment (start 146.2278 95.6404) (end 146.2278 98.3196) (width 0.5) (layer "F.Cu") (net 6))
 (segment (start 148.5773 95.1357) (end 148.1836 95.5294) (width 0.5) (layer "F.Cu") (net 6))
 (segment (start 148.1836 95.5294) (end 146.3388 95.5294) (width 0.5) (layer "F.Cu") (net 6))
 (segment (start 157.2768 90.227) (end 157.353 90.3032) (width 0.5) (layer "F.Cu") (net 6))
 (segment (start 155.2194 90.227) (end 157.2768 90.227) (width 0.5) (layer "F.Cu") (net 6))
 (via (at 155.2194 90.227) (size 0.5) (drill 0.3) (layers "F.Cu" "B.Cu") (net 6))
 (via (at 148.5773 95.1357) (size 0.5) (drill 0.3) (layers "F.Cu" "B.Cu") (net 6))
 (segment (start 155.2194 90.227) (end 153.486 90.227) (width 0.5) (layer "B.Cu") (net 6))
 (segment (start 153.486 90.227) (end 148.5773 95.1357) (width 0.5) (layer "B.Cu") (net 6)))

